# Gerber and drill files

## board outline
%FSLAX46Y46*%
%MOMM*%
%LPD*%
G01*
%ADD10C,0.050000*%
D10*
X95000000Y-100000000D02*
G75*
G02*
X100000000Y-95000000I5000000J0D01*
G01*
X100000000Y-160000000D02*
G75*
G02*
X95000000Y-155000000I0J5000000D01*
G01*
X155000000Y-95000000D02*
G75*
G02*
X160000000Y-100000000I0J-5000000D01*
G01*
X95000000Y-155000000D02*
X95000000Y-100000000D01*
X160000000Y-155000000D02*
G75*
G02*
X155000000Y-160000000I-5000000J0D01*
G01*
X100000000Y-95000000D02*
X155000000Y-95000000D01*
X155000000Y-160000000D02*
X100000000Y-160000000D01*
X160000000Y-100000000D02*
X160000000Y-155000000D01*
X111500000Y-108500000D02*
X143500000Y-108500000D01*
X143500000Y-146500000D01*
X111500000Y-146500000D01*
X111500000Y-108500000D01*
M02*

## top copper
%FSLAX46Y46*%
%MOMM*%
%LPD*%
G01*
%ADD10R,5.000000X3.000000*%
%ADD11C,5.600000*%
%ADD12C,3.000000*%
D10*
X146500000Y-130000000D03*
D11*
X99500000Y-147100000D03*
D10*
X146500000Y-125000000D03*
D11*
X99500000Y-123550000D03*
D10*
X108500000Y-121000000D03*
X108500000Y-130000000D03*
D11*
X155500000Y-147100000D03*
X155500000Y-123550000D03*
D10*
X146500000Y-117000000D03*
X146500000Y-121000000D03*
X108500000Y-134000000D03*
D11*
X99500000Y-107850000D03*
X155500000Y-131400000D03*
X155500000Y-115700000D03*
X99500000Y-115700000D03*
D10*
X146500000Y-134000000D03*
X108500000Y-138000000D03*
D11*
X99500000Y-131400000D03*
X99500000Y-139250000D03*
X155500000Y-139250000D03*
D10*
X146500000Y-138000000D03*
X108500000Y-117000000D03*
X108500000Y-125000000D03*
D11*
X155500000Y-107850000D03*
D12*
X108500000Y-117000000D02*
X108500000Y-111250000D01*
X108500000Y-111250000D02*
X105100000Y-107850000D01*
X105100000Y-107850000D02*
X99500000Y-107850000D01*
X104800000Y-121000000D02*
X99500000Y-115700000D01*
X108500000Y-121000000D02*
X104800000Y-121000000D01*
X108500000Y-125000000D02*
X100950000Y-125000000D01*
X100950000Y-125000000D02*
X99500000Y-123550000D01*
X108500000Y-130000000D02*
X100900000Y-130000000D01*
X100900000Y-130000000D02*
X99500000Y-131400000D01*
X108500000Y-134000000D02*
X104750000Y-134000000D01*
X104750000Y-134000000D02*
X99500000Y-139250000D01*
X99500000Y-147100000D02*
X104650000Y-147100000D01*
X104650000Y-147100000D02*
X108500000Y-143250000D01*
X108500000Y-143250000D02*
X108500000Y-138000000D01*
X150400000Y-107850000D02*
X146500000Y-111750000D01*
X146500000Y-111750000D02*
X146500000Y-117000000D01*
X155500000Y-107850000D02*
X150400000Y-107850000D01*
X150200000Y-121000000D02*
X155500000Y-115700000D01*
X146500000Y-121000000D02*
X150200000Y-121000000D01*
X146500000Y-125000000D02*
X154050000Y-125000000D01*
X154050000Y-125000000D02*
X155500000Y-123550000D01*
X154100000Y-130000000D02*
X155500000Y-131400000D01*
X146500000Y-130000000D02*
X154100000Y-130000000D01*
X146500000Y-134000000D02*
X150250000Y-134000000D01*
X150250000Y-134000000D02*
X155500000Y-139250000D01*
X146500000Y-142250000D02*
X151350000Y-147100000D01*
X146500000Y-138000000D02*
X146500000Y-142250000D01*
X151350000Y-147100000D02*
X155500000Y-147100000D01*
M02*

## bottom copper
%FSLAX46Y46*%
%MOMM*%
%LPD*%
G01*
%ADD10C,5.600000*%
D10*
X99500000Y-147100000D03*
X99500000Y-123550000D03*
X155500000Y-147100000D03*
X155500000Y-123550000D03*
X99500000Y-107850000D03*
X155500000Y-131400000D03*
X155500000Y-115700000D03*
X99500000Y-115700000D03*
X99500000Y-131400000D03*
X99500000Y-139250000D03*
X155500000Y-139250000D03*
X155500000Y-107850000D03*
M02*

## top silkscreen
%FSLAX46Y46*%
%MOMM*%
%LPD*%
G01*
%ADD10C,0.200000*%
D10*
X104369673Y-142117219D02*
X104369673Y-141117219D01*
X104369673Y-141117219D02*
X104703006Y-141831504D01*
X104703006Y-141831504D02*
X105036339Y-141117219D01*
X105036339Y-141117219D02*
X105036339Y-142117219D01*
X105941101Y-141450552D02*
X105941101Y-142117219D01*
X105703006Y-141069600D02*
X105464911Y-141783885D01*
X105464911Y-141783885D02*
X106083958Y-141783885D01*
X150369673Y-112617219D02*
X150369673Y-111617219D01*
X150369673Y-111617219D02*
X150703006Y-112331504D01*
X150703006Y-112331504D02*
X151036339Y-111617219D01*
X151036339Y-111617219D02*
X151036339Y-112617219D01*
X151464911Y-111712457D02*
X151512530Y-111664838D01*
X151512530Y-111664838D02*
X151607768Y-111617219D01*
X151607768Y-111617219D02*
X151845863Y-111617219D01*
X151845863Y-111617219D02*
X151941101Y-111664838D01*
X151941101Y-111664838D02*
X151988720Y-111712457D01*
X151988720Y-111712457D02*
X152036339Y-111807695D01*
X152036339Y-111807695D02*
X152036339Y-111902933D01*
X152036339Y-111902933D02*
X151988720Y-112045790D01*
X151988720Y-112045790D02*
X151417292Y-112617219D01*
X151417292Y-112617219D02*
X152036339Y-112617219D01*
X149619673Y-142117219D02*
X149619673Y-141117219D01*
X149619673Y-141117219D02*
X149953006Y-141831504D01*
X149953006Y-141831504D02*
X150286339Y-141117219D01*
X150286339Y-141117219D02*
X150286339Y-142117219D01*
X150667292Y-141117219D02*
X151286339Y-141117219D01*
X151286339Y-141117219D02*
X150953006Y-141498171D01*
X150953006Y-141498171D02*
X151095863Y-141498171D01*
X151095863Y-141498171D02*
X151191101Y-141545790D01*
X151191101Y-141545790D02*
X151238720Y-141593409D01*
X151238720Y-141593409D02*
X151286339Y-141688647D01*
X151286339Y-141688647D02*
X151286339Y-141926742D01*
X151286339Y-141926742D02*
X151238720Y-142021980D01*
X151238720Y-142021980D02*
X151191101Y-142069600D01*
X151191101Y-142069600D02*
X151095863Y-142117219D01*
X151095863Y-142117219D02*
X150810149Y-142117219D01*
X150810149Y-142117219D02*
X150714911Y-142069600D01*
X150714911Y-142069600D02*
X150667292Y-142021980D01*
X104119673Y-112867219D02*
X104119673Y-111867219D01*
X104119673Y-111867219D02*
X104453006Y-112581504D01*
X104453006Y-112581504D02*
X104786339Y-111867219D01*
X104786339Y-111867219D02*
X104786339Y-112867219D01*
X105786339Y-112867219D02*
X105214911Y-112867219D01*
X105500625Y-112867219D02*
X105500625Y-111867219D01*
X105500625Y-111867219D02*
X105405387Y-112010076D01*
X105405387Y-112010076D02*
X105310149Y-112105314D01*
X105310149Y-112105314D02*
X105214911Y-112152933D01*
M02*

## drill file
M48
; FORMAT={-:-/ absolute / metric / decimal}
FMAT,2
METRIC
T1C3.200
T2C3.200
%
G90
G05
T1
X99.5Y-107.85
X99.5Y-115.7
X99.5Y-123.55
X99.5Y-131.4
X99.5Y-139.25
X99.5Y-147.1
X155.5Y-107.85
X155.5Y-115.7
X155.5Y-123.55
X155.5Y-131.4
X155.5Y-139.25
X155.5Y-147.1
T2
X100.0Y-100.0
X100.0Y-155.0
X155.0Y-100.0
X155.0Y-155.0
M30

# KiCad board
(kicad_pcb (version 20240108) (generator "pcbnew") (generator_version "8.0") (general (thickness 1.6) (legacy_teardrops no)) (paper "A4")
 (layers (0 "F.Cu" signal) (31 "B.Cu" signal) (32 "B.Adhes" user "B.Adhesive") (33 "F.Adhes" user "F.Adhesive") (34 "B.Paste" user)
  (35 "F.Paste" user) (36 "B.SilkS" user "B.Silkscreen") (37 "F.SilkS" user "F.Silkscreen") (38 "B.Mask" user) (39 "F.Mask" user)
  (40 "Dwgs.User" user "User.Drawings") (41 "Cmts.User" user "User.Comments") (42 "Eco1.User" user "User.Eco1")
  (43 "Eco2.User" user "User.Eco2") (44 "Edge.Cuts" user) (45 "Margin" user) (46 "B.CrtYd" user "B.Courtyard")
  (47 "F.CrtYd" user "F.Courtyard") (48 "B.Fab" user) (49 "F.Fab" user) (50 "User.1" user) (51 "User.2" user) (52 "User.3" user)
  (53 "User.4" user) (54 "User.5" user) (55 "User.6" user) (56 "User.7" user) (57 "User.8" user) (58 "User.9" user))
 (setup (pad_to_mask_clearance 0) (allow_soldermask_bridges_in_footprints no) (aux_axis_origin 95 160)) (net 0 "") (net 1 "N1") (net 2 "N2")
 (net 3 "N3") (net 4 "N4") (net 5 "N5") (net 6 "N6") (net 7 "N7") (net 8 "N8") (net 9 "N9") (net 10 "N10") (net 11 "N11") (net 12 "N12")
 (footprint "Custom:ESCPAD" (layer "F.Cu") (at 146.5 130)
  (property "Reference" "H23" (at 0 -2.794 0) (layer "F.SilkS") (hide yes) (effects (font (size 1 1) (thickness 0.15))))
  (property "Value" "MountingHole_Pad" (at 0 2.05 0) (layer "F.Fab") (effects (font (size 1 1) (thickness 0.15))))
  (pad "1" smd rect (at 0 0) (size 5 3) (layers "F.Cu" "F.Mask") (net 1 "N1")))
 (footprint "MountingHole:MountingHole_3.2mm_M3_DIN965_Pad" (layer "F.Cu") (at 99.5 147.1)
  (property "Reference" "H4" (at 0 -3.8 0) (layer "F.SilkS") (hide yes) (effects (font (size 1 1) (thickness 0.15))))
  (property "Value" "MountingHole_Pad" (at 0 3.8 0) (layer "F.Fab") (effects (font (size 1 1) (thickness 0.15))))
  (pad "1" thru_hole circle (at 0 0) (size 5.6 5.6) (drill 3.2) (layers "*.Cu" "*.Mask") (remove_unused_layers no) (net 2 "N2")))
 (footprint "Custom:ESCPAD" (layer "F.Cu") (at 146.5 125)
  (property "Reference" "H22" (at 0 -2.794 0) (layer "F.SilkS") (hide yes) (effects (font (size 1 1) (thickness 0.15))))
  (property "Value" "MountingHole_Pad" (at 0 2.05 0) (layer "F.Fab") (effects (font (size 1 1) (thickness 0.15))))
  (pad "1" smd rect (at 0 0) (size 5 3) (layers "F.Cu" "F.Mask") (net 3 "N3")))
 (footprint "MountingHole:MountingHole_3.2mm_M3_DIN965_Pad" (layer "F.Cu") (at 99.5 123.55)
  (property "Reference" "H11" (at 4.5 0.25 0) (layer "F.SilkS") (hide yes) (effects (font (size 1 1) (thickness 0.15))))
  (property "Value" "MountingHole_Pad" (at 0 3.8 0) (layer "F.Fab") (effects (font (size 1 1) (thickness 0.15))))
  (pad "1" thru_hole circle (at 0 0) (size 5.6 5.6) (drill 3.2) (layers "*.Cu" "*.Mask") (remove_unused_layers no) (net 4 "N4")))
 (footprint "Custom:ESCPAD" (layer "F.Cu") (at 108.5 121)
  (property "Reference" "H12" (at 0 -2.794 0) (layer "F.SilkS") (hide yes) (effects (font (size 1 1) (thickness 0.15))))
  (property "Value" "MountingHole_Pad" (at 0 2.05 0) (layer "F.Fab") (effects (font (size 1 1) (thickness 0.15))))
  (pad "1" smd rect (at 0 0) (size 5 3) (layers "F.Cu" "F.Mask") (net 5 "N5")))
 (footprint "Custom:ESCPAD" (layer "F.Cu") (at 108.5 130)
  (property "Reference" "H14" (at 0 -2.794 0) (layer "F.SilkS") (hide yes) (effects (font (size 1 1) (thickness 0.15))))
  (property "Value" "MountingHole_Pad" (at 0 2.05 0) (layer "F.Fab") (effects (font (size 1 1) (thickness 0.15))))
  (pad "1" smd rect (at 0 0) (size 5 3) (layers "F.Cu" "F.Mask") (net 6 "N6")))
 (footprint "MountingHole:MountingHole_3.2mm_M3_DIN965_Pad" (layer "F.Cu") (at 155.5 147.1)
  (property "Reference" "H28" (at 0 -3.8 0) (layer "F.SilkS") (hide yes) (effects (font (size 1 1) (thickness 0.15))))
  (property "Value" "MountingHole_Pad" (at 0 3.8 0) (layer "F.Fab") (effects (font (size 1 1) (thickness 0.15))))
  (pad "1" thru_hole circle (at 0 0) (size 5.6 5.6) (drill 3.2) (layers "*.Cu" "*.Mask") (remove_unused_layers no) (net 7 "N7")))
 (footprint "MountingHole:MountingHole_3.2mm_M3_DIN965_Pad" (layer "F.Cu") (at 155.5 123.55)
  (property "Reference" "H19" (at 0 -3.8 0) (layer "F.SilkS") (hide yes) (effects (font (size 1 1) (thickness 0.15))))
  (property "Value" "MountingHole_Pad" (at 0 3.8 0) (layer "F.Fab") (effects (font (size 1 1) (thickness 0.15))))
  (pad "1" thru_hole circle (at 0 0) (size 5.6 5.6) (drill 3.2) (layers "*.Cu" "*.Mask") (remove_unused_layers no) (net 3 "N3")))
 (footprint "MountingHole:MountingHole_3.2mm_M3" (layer "F.Cu") (at 155 155)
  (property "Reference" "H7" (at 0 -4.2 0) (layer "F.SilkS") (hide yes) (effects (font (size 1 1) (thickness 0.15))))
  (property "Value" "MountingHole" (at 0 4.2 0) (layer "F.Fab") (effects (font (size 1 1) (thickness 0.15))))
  (pad "" np_thru_hole circle (at 0 0) (size 3.2 3.2) (drill 3.2) (layers "*.Cu" "*.Mask")))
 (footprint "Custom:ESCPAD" (layer "F.Cu") (at 146.5 117)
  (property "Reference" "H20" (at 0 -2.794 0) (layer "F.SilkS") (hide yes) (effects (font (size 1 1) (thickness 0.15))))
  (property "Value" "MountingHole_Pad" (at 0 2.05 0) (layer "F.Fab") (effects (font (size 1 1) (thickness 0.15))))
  (pad "1" smd rect (at 0 0) (size 5 3) (layers "F.Cu" "F.Mask") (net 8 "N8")))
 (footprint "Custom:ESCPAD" (layer "F.Cu") (at 146.5 121)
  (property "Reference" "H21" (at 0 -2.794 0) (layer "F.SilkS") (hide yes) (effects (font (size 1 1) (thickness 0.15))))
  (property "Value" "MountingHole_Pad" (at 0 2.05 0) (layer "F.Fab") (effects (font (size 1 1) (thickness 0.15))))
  (pad "1" smd rect (at 0 0) (size 5 3) (layers "F.Cu" "F.Mask") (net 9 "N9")))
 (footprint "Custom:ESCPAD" (layer "F.Cu") (at 108.5 134)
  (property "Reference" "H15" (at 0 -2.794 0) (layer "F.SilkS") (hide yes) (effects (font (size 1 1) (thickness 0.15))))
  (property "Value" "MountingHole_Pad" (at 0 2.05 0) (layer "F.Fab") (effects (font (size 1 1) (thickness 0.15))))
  (pad "1" smd rect (at 0 0) (size 5 3) (layers "F.Cu" "F.Mask") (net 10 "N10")))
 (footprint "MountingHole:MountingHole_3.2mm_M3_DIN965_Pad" (layer "F.Cu") (at 99.5 107.85)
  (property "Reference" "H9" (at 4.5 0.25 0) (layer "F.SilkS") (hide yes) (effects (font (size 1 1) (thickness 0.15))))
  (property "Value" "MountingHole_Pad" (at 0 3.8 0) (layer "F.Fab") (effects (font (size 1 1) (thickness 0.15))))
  (pad "1" thru_hole circle (at 0 0) (size 5.6 5.6) (drill 3.2) (layers "*.Cu" "*.Mask") (remove_unused_layers no) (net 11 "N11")))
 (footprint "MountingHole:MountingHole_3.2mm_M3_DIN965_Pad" (layer "F.Cu") (at 155.5 131.4)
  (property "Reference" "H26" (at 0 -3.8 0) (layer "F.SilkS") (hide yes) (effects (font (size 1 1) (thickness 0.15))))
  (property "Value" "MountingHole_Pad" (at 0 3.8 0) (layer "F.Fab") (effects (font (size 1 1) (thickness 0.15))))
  (pad "1" thru_hole circle (at 0 0) (size 5.6 5.6) (drill 3.2) (layers "*.Cu" "*.Mask") (remove_unused_layers no) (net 1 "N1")))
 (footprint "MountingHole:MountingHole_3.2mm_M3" (layer "F.Cu") (at 100 155)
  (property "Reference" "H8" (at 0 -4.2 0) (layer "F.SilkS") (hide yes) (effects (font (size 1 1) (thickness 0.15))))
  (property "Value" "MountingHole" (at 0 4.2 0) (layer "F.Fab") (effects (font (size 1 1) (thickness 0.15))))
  (pad "" np_thru_hole circle (at 0 0) (size 3.2 3.2) (drill 3.2) (layers "*.Cu" "*.Mask")))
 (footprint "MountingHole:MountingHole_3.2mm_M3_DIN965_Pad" (layer "F.Cu") (at 155.5 115.7)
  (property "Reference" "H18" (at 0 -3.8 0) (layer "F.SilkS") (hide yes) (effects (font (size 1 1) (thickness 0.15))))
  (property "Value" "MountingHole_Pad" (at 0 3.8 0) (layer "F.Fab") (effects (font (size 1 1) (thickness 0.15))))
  (pad "1" thru_hole circle (at 0 0) (size 5.6 5.6) (drill 3.2) (layers "*.Cu" "*.Mask") (remove_unused_layers no) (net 9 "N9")))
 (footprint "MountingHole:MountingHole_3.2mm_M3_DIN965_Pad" (layer "F.Cu") (at 99.5 115.7)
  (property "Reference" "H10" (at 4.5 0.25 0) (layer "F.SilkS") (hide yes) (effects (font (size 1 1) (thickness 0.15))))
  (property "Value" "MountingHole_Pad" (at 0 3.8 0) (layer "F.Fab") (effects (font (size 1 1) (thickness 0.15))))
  (pad "1" thru_hole circle (at 0 0) (size 5.6 5.6) (drill 3.2) (layers "*.Cu" "*.Mask") (remove_unused_layers no) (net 5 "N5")))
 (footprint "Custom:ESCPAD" (layer "F.Cu") (at 146.5 134)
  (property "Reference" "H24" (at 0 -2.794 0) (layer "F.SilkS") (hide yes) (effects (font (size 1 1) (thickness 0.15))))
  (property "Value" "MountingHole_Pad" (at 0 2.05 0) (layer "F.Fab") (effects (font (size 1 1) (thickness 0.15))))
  (pad "1" smd rect (at 0 0) (size 5 3) (layers "F.Cu" "F.Mask") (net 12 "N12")))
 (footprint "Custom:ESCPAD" (layer "F.Cu") (at 108.5 138)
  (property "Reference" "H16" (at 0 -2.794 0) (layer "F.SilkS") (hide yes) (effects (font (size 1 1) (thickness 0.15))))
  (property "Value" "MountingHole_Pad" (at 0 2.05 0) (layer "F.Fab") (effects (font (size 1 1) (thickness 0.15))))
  (pad "1" smd rect (at 0 0) (size 5 3) (layers "F.Cu" "F.Mask") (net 2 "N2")))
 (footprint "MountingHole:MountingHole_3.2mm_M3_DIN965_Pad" (layer "F.Cu") (at 99.5 131.4)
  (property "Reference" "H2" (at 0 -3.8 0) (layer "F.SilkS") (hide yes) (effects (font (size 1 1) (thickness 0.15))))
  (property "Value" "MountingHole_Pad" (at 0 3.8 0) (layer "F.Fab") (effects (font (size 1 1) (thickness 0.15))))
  (pad "1" thru_hole circle (at 0 0) (size 5.6 5.6) (drill 3.2) (layers "*.Cu" "*.Mask") (remove_unused_layers no) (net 6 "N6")))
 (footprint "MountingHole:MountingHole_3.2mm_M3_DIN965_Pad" (layer "F.Cu") (at 99.5 139.25)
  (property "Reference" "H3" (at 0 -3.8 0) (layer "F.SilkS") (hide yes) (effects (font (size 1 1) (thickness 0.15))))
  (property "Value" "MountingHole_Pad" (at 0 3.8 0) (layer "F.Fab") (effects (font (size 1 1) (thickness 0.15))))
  (pad "1" thru_hole circle (at 0 0) (size 5.6 5.6) (drill 3.2) (layers "*.Cu" "*.Mask") (remove_unused_layers no) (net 10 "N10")))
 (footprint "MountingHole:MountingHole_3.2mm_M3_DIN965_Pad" (layer "F.Cu") (at 155.5 139.25)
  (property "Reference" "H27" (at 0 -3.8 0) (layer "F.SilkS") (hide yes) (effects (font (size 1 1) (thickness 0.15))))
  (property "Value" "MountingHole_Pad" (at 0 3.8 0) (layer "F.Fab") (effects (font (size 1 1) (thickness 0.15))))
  (pad "1" thru_hole circle (at 0 0) (size 5.6 5.6) (drill 3.2) (layers "*.Cu" "*.Mask") (remove_unused_layers no) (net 12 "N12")))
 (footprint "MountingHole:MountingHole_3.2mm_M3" (layer "F.Cu") (at 100 100)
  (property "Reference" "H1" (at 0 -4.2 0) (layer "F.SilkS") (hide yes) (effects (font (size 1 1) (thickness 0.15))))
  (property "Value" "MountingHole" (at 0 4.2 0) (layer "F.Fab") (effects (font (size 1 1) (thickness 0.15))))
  (pad "" np_thru_hole circle (at 0 0) (size 3.2 3.2) (drill 3.2) (layers "*.Cu" "*.Mask")))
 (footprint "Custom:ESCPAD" (layer "F.Cu") (at 146.5 138)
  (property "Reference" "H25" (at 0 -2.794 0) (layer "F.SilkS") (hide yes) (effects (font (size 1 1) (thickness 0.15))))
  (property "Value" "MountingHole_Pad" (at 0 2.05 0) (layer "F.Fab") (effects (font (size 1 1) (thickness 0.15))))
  (pad "1" smd rect (at 0 0) (size 5 3) (layers "F.Cu" "F.Mask") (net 7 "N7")))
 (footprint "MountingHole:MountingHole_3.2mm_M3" (layer "F.Cu") (at 155 100)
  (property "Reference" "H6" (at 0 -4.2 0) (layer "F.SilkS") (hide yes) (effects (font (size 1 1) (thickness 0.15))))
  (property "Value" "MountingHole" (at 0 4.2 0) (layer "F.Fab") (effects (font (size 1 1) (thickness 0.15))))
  (pad "" np_thru_hole circle (at 0 0) (size 3.2 3.2) (drill 3.2) (layers "*.Cu" "*.Mask")))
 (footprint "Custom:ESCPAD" (layer "F.Cu") (at 108.5 117)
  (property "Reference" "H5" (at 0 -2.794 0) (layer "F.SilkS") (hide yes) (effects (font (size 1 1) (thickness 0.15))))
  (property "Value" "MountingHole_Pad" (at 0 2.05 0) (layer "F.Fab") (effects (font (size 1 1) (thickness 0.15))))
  (pad "1" smd rect (at 0 0) (size 5 3) (layers "F.Cu" "F.Mask") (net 11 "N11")))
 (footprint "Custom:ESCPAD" (layer "F.Cu") (at 108.5 125)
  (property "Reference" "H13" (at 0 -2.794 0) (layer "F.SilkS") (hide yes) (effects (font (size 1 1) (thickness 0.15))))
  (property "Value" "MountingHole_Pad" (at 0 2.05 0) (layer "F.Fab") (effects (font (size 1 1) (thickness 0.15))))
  (pad "1" smd rect (at 0 0) (size 5 3) (layers "F.Cu" "F.Mask") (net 4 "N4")))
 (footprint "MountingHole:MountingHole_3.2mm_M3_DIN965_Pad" (layer "F.Cu") (at 155.5 107.85)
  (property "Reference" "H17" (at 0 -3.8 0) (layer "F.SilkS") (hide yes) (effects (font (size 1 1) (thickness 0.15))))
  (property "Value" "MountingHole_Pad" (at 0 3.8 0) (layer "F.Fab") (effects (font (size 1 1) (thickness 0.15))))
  (pad "1" thru_hole circle (at 0 0) (size 5.6 5.6) (drill 3.2) (layers "*.Cu" "*.Mask") (remove_unused_layers no) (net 8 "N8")))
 (gr_arc (start 95 100) (mid 96.464466 96.464466) (end 100 95) (stroke (width 0.05) (type default)) (layer "Edge.Cuts"))
 (gr_arc (start 100 160) (mid 96.464466 158.535534) (end 95 155) (stroke (width 0.05) (type default)) (layer "Edge.Cuts"))
 (gr_arc (start 155 95) (mid 158.535534 96.464466) (end 160 100) (stroke (width 0.05) (type default)) (layer "Edge.Cuts"))
 (gr_line (start 95 155) (end 95 100) (stroke (width 0.05) (type default)) (layer "Edge.Cuts"))
 (gr_arc (start 160 155) (mid 158.535534 158.535534) (end 155 160) (stroke (width 0.05) (type default)) (layer "Edge.Cuts"))
 (gr_line (start 100 95) (end 155 95) (stroke (width 0.05) (type default)) (layer "Edge.Cuts"))
 (gr_line (start 155 160) (end 100 160) (stroke (width 0.05) (type default)) (layer "Edge.Cuts"))
 (gr_line (start 160 100) (end 160 155) (stroke (width 0.05) (type default)) (layer "Edge.Cuts"))
 (gr_rect (start 111.5 108.5) (end 143.5 146.5) (stroke (width 0.05) (type default)) (fill none) (layer "Edge.Cuts"))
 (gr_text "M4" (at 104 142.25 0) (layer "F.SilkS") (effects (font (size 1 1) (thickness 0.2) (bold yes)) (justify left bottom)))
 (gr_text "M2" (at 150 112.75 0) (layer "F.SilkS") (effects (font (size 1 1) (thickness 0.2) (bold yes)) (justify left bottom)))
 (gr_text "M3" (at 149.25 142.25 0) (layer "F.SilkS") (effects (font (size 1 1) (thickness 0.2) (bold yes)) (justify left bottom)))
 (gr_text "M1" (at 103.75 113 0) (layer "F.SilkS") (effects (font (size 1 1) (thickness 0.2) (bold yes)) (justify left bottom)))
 (segment (start 108.5 117) (end 108.5 111.25) (width 3) (layer "F.Cu") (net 11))
 (segment (start 108.5 111.25) (end 105.1 107.85) (width 3) (layer "F.Cu") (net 11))
 (segment (start 105.1 107.85) (end 99.5 107.85) (width 3) (layer "F.Cu") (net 11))
 (segment (start 104.8 121) (end 99.5 115.7) (width 3) (layer "F.Cu") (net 5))
 (segment (start 108.5 121) (end 104.8 121) (width 3) (layer "F.Cu") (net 5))
 (segment (start 108.5 125) (end 100.95 125) (width 3) (layer "F.Cu") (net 4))
 (segment (start 100.95 125) (end 99.5 123.55) (width 3) (layer "F.Cu") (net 4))
 (segment (start 108.5 130) (end 100.9 130) (width 3) (layer "F.Cu") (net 6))
 (segment (start 100.9 130) (end 99.5 131.4) (width 3) (layer "F.Cu") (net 6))
 (segment (start 108.5 134) (end 104.75 134) (width 3) (layer "F.Cu") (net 10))
 (segment (start 104.75 134) (end 99.5 139.25) (width 3) (layer "F.Cu") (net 10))
 (segment (start 99.5 147.1) (end 104.65 147.1) (width 3) (layer "F.Cu") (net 2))
 (segment (start 104.65 147.1) (end 108.5 143.25) (width 3) (layer "F.Cu") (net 2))
 (segment (start 108.5 143.25) (end 108.5 138) (width 3) (layer "F.Cu") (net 2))
 (segment (start 150.4 107.85) (end 146.5 111.75) (width 3) (layer "F.Cu") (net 8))
 (segment (start 146.5 111.75) (end 146.5 117) (width 3) (layer "F.Cu") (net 8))
 (segment (start 155.5 107.85) (end 150.4 107.85) (width 3) (layer "F.Cu") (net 8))
 (segment (start 150.2 121) (end 155.5 115.7) (width 3) (layer "F.Cu") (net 9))
 (segment (start 146.5 121) (end 150.2 121) (width 3) (layer "F.Cu") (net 9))
 (segment (start 146.5 125) (end 154.05 125) (width 3) (layer "F.Cu") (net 3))
 (segment (start 154.05 125) (end 155.5 123.55) (width 3) (layer "F.Cu") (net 3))
 (segment (start 154.1 130) (end 155.5 131.4) (width 3) (layer "F.Cu") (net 1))
 (segment (start 146.5 130) (end 154.1 130) (width 3) (layer "F.Cu") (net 1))
 (segment (start 146.5 134) (end 150.25 134) (width 3) (layer "F.Cu") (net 12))
 (segment (start 150.25 134) (end 155.5 139.25) (width 3) (layer "F.Cu") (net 12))
 (segment (start 146.5 142.25) (end 151.35 147.1) (width 3) (layer "F.Cu") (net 7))
 (segment (start 146.5 138) (end 146.5 142.25) (width 3) (layer "F.Cu") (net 7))
 (segment (start 151.35 147.1) (end 155.5 147.1) (width 3) (layer "F.Cu") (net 7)))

